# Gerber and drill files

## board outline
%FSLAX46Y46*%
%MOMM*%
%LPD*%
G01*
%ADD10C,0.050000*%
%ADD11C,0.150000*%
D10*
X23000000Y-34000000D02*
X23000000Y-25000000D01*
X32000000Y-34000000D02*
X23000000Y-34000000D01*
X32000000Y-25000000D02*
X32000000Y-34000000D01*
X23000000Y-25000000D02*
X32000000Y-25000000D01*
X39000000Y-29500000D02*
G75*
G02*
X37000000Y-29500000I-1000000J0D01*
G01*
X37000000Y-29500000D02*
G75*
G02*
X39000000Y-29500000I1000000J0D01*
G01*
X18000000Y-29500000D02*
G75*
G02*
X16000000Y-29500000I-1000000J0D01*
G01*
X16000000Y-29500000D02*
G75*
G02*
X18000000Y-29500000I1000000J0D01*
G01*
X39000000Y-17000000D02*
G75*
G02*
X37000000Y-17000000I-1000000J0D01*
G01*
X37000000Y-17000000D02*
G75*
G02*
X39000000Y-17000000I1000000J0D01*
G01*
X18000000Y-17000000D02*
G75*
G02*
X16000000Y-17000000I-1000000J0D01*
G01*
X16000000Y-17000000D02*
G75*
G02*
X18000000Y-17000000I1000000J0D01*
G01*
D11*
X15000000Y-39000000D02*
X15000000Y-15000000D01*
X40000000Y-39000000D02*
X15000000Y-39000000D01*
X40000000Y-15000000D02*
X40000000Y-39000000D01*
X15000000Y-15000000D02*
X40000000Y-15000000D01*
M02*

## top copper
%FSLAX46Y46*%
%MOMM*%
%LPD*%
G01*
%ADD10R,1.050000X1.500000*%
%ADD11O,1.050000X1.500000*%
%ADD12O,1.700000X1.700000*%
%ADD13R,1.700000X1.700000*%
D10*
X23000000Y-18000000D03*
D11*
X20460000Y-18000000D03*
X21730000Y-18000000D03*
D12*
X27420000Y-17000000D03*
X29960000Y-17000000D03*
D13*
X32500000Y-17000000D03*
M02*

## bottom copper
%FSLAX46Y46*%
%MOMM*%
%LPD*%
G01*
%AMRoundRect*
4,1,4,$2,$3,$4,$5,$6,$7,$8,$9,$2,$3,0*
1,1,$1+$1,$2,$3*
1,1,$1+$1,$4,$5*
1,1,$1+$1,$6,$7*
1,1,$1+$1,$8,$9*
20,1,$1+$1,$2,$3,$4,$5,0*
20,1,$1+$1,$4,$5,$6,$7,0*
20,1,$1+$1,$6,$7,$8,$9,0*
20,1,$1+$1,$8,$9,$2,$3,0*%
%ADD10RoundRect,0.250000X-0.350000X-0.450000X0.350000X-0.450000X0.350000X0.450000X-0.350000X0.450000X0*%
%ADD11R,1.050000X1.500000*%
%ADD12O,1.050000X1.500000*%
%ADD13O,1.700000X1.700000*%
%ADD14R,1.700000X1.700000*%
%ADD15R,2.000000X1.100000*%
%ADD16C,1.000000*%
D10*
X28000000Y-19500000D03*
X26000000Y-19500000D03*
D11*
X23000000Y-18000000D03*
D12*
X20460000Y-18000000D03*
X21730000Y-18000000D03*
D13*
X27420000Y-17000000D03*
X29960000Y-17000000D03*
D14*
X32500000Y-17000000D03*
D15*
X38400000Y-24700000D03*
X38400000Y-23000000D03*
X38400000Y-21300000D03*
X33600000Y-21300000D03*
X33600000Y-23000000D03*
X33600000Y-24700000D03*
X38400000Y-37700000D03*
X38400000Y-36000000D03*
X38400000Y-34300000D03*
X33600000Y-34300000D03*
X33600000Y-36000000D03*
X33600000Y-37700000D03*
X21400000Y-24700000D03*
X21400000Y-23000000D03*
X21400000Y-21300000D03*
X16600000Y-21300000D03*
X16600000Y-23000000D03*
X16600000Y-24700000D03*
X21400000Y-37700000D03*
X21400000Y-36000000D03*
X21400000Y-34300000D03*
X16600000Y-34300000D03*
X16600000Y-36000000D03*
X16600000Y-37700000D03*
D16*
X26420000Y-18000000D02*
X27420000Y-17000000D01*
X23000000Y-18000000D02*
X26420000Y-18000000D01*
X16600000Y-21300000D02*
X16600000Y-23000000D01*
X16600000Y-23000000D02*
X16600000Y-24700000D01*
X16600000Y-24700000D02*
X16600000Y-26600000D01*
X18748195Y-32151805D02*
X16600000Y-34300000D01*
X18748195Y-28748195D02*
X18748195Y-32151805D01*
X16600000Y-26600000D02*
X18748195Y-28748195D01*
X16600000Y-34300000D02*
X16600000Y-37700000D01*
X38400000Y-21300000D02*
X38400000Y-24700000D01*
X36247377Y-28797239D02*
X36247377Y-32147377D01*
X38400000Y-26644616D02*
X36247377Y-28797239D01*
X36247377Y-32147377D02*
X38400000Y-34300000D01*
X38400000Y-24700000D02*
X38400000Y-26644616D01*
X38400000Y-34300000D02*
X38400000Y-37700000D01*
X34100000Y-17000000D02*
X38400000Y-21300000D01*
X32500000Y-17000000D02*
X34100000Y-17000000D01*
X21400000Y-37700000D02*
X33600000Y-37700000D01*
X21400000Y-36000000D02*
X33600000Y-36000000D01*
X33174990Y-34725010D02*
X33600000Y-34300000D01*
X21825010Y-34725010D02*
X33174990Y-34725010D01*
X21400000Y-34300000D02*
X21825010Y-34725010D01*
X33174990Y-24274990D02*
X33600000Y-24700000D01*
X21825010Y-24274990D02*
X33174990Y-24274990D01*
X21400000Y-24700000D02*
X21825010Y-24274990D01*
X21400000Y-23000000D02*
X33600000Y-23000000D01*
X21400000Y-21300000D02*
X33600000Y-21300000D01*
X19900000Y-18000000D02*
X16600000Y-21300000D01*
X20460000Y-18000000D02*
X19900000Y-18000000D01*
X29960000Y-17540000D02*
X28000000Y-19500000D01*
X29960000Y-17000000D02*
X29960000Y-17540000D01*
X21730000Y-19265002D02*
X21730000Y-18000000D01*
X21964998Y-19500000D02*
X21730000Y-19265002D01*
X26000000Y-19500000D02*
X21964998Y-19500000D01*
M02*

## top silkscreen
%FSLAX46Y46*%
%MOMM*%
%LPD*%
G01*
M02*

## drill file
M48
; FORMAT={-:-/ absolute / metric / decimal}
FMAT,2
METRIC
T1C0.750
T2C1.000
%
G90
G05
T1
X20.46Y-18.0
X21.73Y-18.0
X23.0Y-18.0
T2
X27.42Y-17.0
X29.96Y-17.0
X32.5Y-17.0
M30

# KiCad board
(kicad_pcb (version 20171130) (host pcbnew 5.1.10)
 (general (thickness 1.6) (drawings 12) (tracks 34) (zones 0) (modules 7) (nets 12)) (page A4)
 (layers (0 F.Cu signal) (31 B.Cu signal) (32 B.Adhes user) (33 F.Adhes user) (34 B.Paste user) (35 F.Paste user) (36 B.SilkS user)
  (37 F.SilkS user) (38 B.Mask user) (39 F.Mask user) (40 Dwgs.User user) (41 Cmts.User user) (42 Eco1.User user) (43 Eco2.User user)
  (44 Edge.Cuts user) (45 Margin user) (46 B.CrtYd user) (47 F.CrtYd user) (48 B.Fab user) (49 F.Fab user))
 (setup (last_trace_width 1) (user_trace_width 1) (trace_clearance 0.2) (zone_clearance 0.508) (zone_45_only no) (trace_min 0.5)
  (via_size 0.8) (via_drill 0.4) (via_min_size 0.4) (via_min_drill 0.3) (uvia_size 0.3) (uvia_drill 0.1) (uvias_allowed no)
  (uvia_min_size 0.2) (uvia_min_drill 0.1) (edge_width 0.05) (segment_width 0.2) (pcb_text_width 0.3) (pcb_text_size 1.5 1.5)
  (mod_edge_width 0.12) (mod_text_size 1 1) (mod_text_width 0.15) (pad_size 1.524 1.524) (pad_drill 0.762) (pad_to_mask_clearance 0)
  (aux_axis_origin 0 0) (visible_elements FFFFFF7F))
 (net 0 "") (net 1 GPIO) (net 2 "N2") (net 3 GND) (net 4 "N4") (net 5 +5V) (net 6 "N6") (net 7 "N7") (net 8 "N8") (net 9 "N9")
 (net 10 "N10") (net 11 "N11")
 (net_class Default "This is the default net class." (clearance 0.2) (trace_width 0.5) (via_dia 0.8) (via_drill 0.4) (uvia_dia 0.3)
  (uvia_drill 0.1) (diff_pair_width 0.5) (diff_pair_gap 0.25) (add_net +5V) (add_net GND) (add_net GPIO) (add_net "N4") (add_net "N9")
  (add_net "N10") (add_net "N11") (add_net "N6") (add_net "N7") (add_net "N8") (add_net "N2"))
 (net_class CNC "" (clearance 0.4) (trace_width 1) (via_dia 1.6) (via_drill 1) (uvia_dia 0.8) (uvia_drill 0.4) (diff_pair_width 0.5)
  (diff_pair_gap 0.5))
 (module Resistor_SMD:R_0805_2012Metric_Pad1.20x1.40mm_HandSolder (layer B.Cu) (at 27 19.5)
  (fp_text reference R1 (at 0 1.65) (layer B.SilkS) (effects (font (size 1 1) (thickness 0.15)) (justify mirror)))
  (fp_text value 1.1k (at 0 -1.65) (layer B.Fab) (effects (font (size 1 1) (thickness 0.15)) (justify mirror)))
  (pad 2 smd roundrect (at 1 0) (size 1.2 1.4) (layers B.Cu B.Paste B.Mask) (roundrect_rratio 0.208333) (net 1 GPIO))
  (pad 1 smd roundrect (at -1 0) (size 1.2 1.4) (layers B.Cu B.Paste B.Mask) (roundrect_rratio 0.208333) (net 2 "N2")))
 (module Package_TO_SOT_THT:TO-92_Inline (layer B.Cu) (at 23 18 180)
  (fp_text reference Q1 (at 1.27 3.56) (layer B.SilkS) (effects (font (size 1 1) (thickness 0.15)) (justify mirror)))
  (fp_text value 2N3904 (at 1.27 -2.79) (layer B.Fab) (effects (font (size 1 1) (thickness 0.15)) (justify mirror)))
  (pad 1 thru_hole rect (at 0 0 180) (size 1.05 1.5) (drill 0.75) (layers *.Cu *.Mask) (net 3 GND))
  (pad 3 thru_hole oval (at 2.54 0 180) (size 1.05 1.5) (drill 0.75) (layers *.Cu *.Mask) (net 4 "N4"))
  (pad 2 thru_hole oval (at 1.27 0 180) (size 1.05 1.5) (drill 0.75) (layers *.Cu *.Mask) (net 2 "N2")))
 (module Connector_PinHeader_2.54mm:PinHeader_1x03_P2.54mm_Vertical (layer B.Cu) (at 32.5 17 90)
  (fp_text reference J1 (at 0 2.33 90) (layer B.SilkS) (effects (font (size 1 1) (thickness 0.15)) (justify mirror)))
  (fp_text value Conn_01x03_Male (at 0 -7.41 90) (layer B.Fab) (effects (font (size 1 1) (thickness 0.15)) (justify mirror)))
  (pad 3 thru_hole oval (at 0 -5.08 90) (size 1.7 1.7) (drill 1) (layers *.Cu *.Mask) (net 3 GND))
  (pad 2 thru_hole oval (at 0 -2.54 90) (size 1.7 1.7) (drill 1) (layers *.Cu *.Mask) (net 1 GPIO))
  (pad 1 thru_hole rect (at 0 0 90) (size 1.7 1.7) (drill 1) (layers *.Cu *.Mask) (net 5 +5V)))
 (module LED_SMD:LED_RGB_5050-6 (layer B.Cu) (at 36 23)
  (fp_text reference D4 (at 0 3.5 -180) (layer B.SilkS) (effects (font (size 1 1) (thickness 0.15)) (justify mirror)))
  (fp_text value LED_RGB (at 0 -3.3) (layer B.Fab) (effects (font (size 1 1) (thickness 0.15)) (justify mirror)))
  (pad 6 smd rect (at 2.4 1.7 270) (size 1.1 2) (layers B.Cu B.Paste B.Mask) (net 5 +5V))
  (pad 5 smd rect (at 2.4 0 270) (size 1.1 2) (layers B.Cu B.Paste B.Mask) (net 5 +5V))
  (pad 4 smd rect (at 2.4 -1.7 270) (size 1.1 2) (layers B.Cu B.Paste B.Mask) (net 5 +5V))
  (pad 3 smd rect (at -2.4 -1.7 270) (size 1.1 2) (layers B.Cu B.Paste B.Mask) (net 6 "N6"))
  (pad 2 smd rect (at -2.4 0 270) (size 1.1 2) (layers B.Cu B.Paste B.Mask) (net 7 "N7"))
  (pad 1 smd rect (at -2.4 1.7 270) (size 1.1 2) (layers B.Cu B.Paste B.Mask) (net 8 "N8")))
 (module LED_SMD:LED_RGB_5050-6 (layer B.Cu) (at 36 36)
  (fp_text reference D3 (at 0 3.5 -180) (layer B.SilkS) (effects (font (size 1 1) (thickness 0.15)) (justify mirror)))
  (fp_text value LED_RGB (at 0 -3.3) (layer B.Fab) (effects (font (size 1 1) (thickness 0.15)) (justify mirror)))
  (pad 6 smd rect (at 2.4 1.7 270) (size 1.1 2) (layers B.Cu B.Paste B.Mask) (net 5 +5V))
  (pad 5 smd rect (at 2.4 0 270) (size 1.1 2) (layers B.Cu B.Paste B.Mask) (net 5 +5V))
  (pad 4 smd rect (at 2.4 -1.7 270) (size 1.1 2) (layers B.Cu B.Paste B.Mask) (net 5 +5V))
  (pad 3 smd rect (at -2.4 -1.7 270) (size 1.1 2) (layers B.Cu B.Paste B.Mask) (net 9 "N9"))
  (pad 2 smd rect (at -2.4 0 270) (size 1.1 2) (layers B.Cu B.Paste B.Mask) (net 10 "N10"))
  (pad 1 smd rect (at -2.4 1.7 270) (size 1.1 2) (layers B.Cu B.Paste B.Mask) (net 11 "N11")))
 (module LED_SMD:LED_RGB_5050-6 (layer B.Cu) (at 19 23)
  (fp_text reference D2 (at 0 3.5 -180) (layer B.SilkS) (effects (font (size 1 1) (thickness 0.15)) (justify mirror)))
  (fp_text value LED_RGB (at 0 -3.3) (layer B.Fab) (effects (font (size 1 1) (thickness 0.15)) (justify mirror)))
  (pad 6 smd rect (at 2.4 1.7 270) (size 1.1 2) (layers B.Cu B.Paste B.Mask) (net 8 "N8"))
  (pad 5 smd rect (at 2.4 0 270) (size 1.1 2) (layers B.Cu B.Paste B.Mask) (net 7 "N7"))
  (pad 4 smd rect (at 2.4 -1.7 270) (size 1.1 2) (layers B.Cu B.Paste B.Mask) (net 6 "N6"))
  (pad 3 smd rect (at -2.4 -1.7 270) (size 1.1 2) (layers B.Cu B.Paste B.Mask) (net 4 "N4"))
  (pad 2 smd rect (at -2.4 0 270) (size 1.1 2) (layers B.Cu B.Paste B.Mask) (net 4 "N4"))
  (pad 1 smd rect (at -2.4 1.7 270) (size 1.1 2) (layers B.Cu B.Paste B.Mask) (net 4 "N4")))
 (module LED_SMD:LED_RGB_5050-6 (layer B.Cu) (at 19 36)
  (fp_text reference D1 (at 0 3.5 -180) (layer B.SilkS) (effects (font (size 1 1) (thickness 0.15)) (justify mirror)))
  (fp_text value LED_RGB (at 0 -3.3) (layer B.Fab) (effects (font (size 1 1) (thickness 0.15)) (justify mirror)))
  (pad 6 smd rect (at 2.4 1.7 270) (size 1.1 2) (layers B.Cu B.Paste B.Mask) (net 11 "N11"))
  (pad 5 smd rect (at 2.4 0 270) (size 1.1 2) (layers B.Cu B.Paste B.Mask) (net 10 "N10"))
  (pad 4 smd rect (at 2.4 -1.7 270) (size 1.1 2) (layers B.Cu B.Paste B.Mask) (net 9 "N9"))
  (pad 3 smd rect (at -2.4 -1.7 270) (size 1.1 2) (layers B.Cu B.Paste B.Mask) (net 4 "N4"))
  (pad 2 smd rect (at -2.4 0 270) (size 1.1 2) (layers B.Cu B.Paste B.Mask) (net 4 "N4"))
  (pad 1 smd rect (at -2.4 1.7 270) (size 1.1 2) (layers B.Cu B.Paste B.Mask) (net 4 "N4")))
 (gr_line (start 23 34) (end 23 25) (layer Edge.Cuts) (width 0.05))
 (gr_line (start 32 34) (end 23 34) (layer Edge.Cuts) (width 0.05))
 (gr_line (start 32 25) (end 32 34) (layer Edge.Cuts) (width 0.05))
 (gr_line (start 23 25) (end 32 25) (layer Edge.Cuts) (width 0.05))
 (gr_circle (center 38 29.5) (end 39 29.5) (layer Edge.Cuts) (width 0.05))
 (gr_circle (center 17 29.5) (end 18 29.5) (layer Edge.Cuts) (width 0.05))
 (gr_circle (center 38 17) (end 39 17) (layer Edge.Cuts) (width 0.05))
 (gr_circle (center 17 17) (end 18 17) (layer Edge.Cuts) (width 0.05))
 (gr_line (start 15 39) (end 15 15) (layer Edge.Cuts) (width 0.15))
 (gr_line (start 40 39) (end 15 39) (layer Edge.Cuts) (width 0.15))
 (gr_line (start 40 15) (end 40 39) (layer Edge.Cuts) (width 0.15))
 (gr_line (start 15 15) (end 40 15) (layer Edge.Cuts) (width 0.15))
 (segment (start 26.42 18) (end 27.42 17) (width 1) (layer B.Cu) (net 3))
 (segment (start 23 18) (end 26.42 18) (width 1) (layer B.Cu) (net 3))
 (segment (start 16.6 21.3) (end 16.6 23) (width 1) (layer B.Cu) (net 4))
 (segment (start 16.6 23) (end 16.6 24.7) (width 1) (layer B.Cu) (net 4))
 (segment (start 16.6 24.7) (end 16.6 26.6) (width 1) (layer B.Cu) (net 4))
 (segment (start 18.748195 32.151805) (end 16.6 34.3) (width 1) (layer B.Cu) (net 4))
 (segment (start 18.748195 28.748195) (end 18.748195 32.151805) (width 1) (layer B.Cu) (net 4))
 (segment (start 16.6 26.6) (end 18.748195 28.748195) (width 1) (layer B.Cu) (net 4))
 (segment (start 16.6 34.3) (end 16.6 37.7) (width 1) (layer B.Cu) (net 4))
 (segment (start 38.4 21.3) (end 38.4 24.7) (width 1) (layer B.Cu) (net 5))
 (segment (start 36.247377 28.797239) (end 36.247377 32.147377) (width 1) (layer B.Cu) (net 5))
 (segment (start 38.4 26.644616) (end 36.247377 28.797239) (width 1) (layer B.Cu) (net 5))
 (segment (start 36.247377 32.147377) (end 38.4 34.3) (width 1) (layer B.Cu) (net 5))
 (segment (start 38.4 24.7) (end 38.4 26.644616) (width 1) (layer B.Cu) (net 5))
 (segment (start 38.4 34.3) (end 38.4 37.7) (width 1) (layer B.Cu) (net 5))
 (segment (start 34.1 17) (end 38.4 21.3) (width 1) (layer B.Cu) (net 5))
 (segment (start 32.5 17) (end 34.1 17) (width 1) (layer B.Cu) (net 5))
 (segment (start 21.4 37.7) (end 33.6 37.7) (width 1) (layer B.Cu) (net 11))
 (segment (start 21.4 36) (end 33.6 36) (width 1) (layer B.Cu) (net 10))
 (segment (start 33.17499 34.72501) (end 33.6 34.3) (width 1) (layer B.Cu) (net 9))
 (segment (start 21.82501 34.72501) (end 33.17499 34.72501) (width 1) (layer B.Cu) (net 9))
 (segment (start 21.4 34.3) (end 21.82501 34.72501) (width 1) (layer B.Cu) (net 9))
 (segment (start 33.17499 24.27499) (end 33.6 24.7) (width 1) (layer B.Cu) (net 8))
 (segment (start 21.82501 24.27499) (end 33.17499 24.27499) (width 1) (layer B.Cu) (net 8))
 (segment (start 21.4 24.7) (end 21.82501 24.27499) (width 1) (layer B.Cu) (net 8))
 (segment (start 21.4 23) (end 33.6 23) (width 1) (layer B.Cu) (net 7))
 (segment (start 21.4 21.3) (end 33.6 21.3) (width 1) (layer B.Cu) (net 6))
 (segment (start 19.9 18) (end 16.6 21.3) (width 1) (layer B.Cu) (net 4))
 (segment (start 20.46 18) (end 19.9 18) (width 1) (layer B.Cu) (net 4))
 (segment (start 29.96 17.54) (end 28 19.5) (width 1) (layer B.Cu) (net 1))
 (segment (start 29.96 17) (end 29.96 17.54) (width 1) (layer B.Cu) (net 1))
 (segment (start 21.73 19.265002) (end 21.73 18) (width 1) (layer B.Cu) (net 2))
 (segment (start 21.964998 19.5) (end 21.73 19.265002) (width 1) (layer B.Cu) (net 2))
 (segment (start 26 19.5) (end 21.964998 19.5) (width 1) (layer B.Cu) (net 2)))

